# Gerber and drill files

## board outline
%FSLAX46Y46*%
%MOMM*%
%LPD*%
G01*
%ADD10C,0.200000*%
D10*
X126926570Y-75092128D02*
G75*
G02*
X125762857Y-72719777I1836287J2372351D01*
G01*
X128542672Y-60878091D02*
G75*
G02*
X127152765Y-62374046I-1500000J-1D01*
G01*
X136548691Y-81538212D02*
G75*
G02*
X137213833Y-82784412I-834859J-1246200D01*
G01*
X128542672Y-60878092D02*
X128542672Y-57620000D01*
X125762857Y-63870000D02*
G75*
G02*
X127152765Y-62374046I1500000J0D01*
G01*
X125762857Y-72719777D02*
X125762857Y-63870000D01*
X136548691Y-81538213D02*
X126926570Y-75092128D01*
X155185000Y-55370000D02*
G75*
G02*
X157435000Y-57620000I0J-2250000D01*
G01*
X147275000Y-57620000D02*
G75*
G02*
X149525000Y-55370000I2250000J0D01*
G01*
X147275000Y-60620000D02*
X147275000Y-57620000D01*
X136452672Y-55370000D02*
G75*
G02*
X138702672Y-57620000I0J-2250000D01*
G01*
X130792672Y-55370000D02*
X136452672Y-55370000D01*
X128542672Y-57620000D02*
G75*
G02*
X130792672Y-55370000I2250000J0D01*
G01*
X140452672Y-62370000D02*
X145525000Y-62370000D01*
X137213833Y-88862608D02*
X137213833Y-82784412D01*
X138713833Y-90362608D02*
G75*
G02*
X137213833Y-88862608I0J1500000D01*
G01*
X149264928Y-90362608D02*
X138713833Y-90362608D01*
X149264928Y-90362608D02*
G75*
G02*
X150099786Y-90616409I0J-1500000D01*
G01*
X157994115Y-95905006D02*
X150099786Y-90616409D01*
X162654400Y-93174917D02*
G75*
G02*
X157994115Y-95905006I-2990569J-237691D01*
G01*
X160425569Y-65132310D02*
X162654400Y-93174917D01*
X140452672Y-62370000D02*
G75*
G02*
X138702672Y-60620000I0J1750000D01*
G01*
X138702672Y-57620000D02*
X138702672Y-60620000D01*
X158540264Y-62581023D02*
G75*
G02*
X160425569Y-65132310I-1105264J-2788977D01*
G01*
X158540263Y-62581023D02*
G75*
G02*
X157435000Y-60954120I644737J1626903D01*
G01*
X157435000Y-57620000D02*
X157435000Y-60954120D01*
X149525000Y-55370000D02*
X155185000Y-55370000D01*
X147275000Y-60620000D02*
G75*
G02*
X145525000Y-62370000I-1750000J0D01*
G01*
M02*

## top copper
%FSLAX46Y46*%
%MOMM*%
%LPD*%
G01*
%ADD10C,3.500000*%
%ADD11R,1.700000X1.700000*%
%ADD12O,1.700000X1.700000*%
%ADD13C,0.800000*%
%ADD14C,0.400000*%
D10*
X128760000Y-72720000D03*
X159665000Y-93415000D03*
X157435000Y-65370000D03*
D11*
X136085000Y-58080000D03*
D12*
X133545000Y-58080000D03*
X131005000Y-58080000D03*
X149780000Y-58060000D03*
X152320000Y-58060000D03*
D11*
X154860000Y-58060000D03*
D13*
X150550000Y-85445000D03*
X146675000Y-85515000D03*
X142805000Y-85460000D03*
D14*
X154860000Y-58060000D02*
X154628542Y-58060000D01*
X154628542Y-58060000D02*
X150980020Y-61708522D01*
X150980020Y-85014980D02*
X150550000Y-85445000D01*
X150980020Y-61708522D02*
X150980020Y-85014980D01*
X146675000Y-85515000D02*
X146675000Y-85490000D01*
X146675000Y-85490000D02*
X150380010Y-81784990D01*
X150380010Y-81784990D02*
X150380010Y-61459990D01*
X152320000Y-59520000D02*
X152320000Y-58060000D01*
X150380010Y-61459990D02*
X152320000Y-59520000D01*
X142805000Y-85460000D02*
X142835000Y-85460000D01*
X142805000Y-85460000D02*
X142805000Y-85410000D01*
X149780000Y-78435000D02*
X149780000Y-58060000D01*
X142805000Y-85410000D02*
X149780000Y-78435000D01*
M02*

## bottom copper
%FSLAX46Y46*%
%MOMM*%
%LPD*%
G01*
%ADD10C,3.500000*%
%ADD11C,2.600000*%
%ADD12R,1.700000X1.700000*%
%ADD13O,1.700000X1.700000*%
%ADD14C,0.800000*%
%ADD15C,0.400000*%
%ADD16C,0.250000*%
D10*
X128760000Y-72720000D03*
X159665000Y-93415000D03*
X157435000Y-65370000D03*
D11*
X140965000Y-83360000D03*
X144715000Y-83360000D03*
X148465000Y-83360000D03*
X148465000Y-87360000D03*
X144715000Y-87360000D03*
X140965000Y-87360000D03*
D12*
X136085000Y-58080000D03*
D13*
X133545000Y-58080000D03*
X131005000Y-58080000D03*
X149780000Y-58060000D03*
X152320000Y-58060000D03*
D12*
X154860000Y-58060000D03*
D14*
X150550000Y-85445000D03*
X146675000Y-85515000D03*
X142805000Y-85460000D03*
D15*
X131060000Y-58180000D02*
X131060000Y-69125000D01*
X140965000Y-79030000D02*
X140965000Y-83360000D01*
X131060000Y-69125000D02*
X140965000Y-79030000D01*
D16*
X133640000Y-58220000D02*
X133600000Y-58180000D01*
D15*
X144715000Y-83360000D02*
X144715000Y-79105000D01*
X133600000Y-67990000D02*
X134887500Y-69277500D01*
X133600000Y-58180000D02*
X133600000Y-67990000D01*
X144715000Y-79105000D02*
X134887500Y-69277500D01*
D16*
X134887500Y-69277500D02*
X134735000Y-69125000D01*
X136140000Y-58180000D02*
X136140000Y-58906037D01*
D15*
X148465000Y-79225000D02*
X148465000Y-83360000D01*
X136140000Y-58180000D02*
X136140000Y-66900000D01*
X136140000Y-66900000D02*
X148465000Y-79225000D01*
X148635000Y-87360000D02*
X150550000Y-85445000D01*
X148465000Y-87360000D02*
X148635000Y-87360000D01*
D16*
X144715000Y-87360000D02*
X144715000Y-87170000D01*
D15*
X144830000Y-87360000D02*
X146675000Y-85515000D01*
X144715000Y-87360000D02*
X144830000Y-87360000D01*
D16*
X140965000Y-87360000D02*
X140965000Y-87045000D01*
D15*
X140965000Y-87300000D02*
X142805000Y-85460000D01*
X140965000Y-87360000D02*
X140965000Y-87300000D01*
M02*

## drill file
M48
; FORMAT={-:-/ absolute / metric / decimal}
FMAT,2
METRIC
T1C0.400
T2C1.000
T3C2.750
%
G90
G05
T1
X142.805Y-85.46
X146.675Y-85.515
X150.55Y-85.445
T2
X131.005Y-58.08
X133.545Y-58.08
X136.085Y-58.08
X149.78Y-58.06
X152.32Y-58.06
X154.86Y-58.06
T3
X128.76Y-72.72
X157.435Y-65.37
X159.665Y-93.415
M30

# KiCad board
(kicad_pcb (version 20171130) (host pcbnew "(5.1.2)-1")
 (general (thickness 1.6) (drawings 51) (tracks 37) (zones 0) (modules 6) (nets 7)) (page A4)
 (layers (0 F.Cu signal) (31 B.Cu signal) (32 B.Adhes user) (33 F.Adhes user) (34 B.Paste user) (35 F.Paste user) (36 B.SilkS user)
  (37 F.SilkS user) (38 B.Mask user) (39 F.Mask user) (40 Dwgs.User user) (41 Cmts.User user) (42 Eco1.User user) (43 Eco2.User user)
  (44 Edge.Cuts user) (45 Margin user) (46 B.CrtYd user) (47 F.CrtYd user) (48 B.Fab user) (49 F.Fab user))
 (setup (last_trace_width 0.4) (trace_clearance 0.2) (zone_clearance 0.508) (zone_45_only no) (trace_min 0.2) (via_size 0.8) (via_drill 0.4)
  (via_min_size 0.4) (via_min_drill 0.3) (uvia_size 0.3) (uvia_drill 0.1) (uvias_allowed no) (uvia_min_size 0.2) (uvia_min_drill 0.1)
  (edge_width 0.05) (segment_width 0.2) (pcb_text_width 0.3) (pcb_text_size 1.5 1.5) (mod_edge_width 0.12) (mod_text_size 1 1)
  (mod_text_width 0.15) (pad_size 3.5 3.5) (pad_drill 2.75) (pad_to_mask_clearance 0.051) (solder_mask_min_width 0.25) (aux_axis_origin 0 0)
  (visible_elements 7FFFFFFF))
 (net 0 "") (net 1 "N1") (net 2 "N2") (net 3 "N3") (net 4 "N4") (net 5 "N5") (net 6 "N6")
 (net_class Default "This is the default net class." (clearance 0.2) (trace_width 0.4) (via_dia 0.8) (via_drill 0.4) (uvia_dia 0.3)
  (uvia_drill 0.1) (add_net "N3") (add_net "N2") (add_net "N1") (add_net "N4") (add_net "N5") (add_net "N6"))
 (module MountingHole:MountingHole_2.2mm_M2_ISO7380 (layer F.Cu) (at 128.76 72.72)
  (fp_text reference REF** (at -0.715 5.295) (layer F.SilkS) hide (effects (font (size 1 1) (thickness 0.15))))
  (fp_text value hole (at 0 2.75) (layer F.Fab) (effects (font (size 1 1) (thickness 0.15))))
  (pad "" np_thru_hole circle (at 0 0) (size 3.5 3.5) (drill 2.75) (layers *.Cu *.Mask)))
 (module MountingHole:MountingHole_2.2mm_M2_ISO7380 (layer F.Cu) (at 159.665 93.415)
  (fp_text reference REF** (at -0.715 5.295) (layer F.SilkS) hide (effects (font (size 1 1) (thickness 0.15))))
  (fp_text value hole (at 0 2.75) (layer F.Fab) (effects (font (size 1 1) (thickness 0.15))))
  (pad "" np_thru_hole circle (at 0 0) (size 3.5 3.5) (drill 2.75) (layers *.Cu *.Mask)))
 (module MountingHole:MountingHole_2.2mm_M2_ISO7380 (layer F.Cu) (at 157.435 65.37)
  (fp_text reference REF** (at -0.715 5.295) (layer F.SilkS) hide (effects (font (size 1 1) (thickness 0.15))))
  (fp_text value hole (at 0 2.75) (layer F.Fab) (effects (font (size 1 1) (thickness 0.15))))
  (pad "" np_thru_hole circle (at 0 0) (size 3.5 3.5) (drill 2.75) (layers *.Cu *.Mask)))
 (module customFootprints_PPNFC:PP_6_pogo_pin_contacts (layer B.Cu) (at 148.465 83.36 180)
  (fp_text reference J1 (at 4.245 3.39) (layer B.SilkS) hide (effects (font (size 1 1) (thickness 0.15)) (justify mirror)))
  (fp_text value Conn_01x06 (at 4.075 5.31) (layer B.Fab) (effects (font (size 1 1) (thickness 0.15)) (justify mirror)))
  (pad 3 smd circle (at 7.5 0 180) (size 2.6 2.6) (layers B.Cu B.Paste B.Mask) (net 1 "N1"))
  (pad 2 smd circle (at 3.75 0 180) (size 2.6 2.6) (layers B.Cu B.Paste B.Mask) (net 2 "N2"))
  (pad 1 smd circle (at 0 0 180) (size 2.6 2.6) (layers B.Cu B.Paste B.Mask) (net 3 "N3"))
  (pad 4 smd circle (at 0 -4 180) (size 2.6 2.6) (layers B.Cu B.Paste B.Mask) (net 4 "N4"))
  (pad 5 smd circle (at 3.75 -4 180) (size 2.6 2.6) (layers B.Cu B.Paste B.Mask) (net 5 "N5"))
  (pad 6 smd circle (at 7.5 -4 180) (size 2.6 2.6) (layers B.Cu B.Paste B.Mask) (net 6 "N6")))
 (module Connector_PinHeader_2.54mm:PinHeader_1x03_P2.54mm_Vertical (layer F.Cu) (at 136.085 58.08 270)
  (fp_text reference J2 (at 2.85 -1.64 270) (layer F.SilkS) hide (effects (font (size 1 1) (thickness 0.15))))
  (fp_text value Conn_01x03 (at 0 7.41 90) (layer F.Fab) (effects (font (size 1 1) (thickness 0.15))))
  (pad 1 thru_hole rect (at 0 0 270) (size 1.7 1.7) (drill 1) (layers *.Cu *.Mask) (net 3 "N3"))
  (pad 2 thru_hole oval (at 0 2.54 270) (size 1.7 1.7) (drill 1) (layers *.Cu *.Mask) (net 2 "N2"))
  (pad 3 thru_hole oval (at 0 5.08 270) (size 1.7 1.7) (drill 1) (layers *.Cu *.Mask) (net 1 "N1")))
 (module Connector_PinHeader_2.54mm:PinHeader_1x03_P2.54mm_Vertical (layer F.Cu) (at 154.86 58.06 270)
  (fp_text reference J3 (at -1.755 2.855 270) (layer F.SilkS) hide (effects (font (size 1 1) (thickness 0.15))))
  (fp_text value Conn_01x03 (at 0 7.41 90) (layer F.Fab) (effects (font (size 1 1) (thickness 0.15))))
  (pad 3 thru_hole oval (at 0 5.08 270) (size 1.7 1.7) (drill 1) (layers *.Cu *.Mask) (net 6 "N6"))
  (pad 2 thru_hole oval (at 0 2.54 270) (size 1.7 1.7) (drill 1) (layers *.Cu *.Mask) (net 5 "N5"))
  (pad 1 thru_hole rect (at 0 0 270) (size 1.7 1.7) (drill 1) (layers *.Cu *.Mask) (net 4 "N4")))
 (gr_arc (start 128.762857 72.719777) (end 125.762857 72.719777) (angle -52.25880262) (layer Edge.Cuts) (width 0.2))
 (gr_arc (start 127.042672 60.878092) (end 127.152765 62.374046) (angle -85.79099191) (layer Edge.Cuts) (width 0.2))
 (gr_arc (start 135.713832 82.784412) (end 137.213833 82.784412) (angle -56.18093969) (layer Edge.Cuts) (width 0.2))
 (gr_line (start 128.542672 60.878092) (end 128.542672 57.62) (layer Edge.Cuts) (width 0.2))
 (gr_arc (start 127.262857 63.87) (end 127.152765 62.374046) (angle -85.79099191) (layer Edge.Cuts) (width 0.2))
 (gr_line (start 125.762857 72.719777) (end 125.762857 63.87) (layer Edge.Cuts) (width 0.2))
 (gr_line (start 136.548691 81.538213) (end 126.92657 75.092128) (layer Edge.Cuts) (width 0.2))
 (gr_arc (start 155.185 57.62) (end 157.435 57.62) (angle -90) (layer Edge.Cuts) (width 0.2))
 (gr_arc (start 149.525 57.62) (end 149.525 55.37) (angle -90) (layer Edge.Cuts) (width 0.2))
 (gr_line (start 147.275 60.62) (end 147.275 57.62) (layer Edge.Cuts) (width 0.2))
 (gr_arc (start 136.452672 57.62) (end 138.702672 57.62) (angle -90) (layer Edge.Cuts) (width 0.2))
 (gr_line (start 130.792672 55.37) (end 136.452672 55.37) (layer Edge.Cuts) (width 0.2))
 (gr_arc (start 130.792672 57.62) (end 130.792672 55.37) (angle -90) (layer Edge.Cuts) (width 0.2))
 (gr_line (start 140.452672 62.37) (end 145.525 62.37) (layer Edge.Cuts) (width 0.2))
 (gr_line (start 137.213833 88.862608) (end 137.213833 82.784412) (layer Edge.Cuts) (width 0.2))
 (gr_arc (start 138.713833 88.862608) (end 137.213833 88.862608) (angle -90) (layer Edge.Cuts) (width 0.2))
 (gr_line (start 149.264928 90.362608) (end 138.713833 90.362608) (layer Edge.Cuts) (width 0.2))
 (gr_arc (start 149.264928 91.862608) (end 150.099786 90.616409) (angle -33.81906031) (layer Edge.Cuts) (width 0.2))
 (gr_line (start 157.994115 95.905006) (end 150.099786 90.616409) (layer Edge.Cuts) (width 0.2))
 (gr_arc (start 159.663831 93.412608) (end 157.994115 95.905006) (angle -128.3633848) (layer Edge.Cuts) (width 0.2))
 (gr_line (start 160.425569 65.13231) (end 162.6544 93.174917) (layer Edge.Cuts) (width 0.2))
 (gr_arc (start 140.452672 60.62) (end 138.702672 60.62) (angle -90) (layer Edge.Cuts) (width 0.2))
 (gr_line (start 138.702672 57.62) (end 138.702672 60.62) (layer Edge.Cuts) (width 0.2))
 (gr_arc (start 157.435 65.37) (end 160.425569 65.13231) (angle -63.83740313) (layer Edge.Cuts) (width 0.2))
 (gr_arc (start 159.185 60.95412) (end 157.435 60.95412) (angle -68.38172758) (layer Edge.Cuts) (width 0.2))
 (gr_line (start 157.435 57.62) (end 157.435 60.95412) (layer Edge.Cuts) (width 0.2))
 (gr_line (start 149.525 55.37) (end 155.185 55.37) (layer Edge.Cuts) (width 0.2))
 (gr_arc (start 145.525 60.62) (end 145.525 62.37) (angle -90) (layer Edge.Cuts) (width 0.2))
 (segment (start 131.06 58.18) (end 131.06 69.125) (width 0.4) (layer B.Cu) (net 1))
 (segment (start 140.965 79.03) (end 140.965 83.36) (width 0.4) (layer B.Cu) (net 1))
 (segment (start 131.06 69.125) (end 140.965 79.03) (width 0.4) (layer B.Cu) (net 1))
 (segment (start 133.64 58.22) (end 133.6 58.18) (width 0.25) (layer B.Cu) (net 2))
 (segment (start 144.715 83.36) (end 144.715 79.105) (width 0.4) (layer B.Cu) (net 2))
 (segment (start 133.6 67.99) (end 134.8875 69.2775) (width 0.4) (layer B.Cu) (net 2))
 (segment (start 133.6 58.18) (end 133.6 67.99) (width 0.4) (layer B.Cu) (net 2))
 (segment (start 144.715 79.105) (end 134.8875 69.2775) (width 0.4) (layer B.Cu) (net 2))
 (segment (start 134.8875 69.2775) (end 134.735 69.125) (width 0.25) (layer B.Cu) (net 2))
 (segment (start 136.14 58.18) (end 136.14 58.906037) (width 0.25) (layer B.Cu) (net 3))
 (segment (start 148.465 79.225) (end 148.465 83.36) (width 0.4) (layer B.Cu) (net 3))
 (segment (start 136.14 58.18) (end 136.14 66.9) (width 0.4) (layer B.Cu) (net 3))
 (segment (start 136.14 66.9) (end 148.465 79.225) (width 0.4) (layer B.Cu) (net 3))
 (via (at 150.55 85.445) (size 0.8) (drill 0.4) (layers F.Cu B.Cu) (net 4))
 (segment (start 148.635 87.36) (end 150.55 85.445) (width 0.4) (layer B.Cu) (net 4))
 (segment (start 148.465 87.36) (end 148.635 87.36) (width 0.4) (layer B.Cu) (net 4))
 (segment (start 154.86 58.06) (end 154.628542 58.06) (width 0.4) (layer F.Cu) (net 4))
 (segment (start 154.628542 58.06) (end 150.98002 61.708522) (width 0.4) (layer F.Cu) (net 4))
 (segment (start 150.98002 85.01498) (end 150.55 85.445) (width 0.4) (layer F.Cu) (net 4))
 (segment (start 150.98002 61.708522) (end 150.98002 85.01498) (width 0.4) (layer F.Cu) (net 4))
 (via (at 146.675 85.515) (size 0.8) (drill 0.4) (layers F.Cu B.Cu) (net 5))
 (segment (start 144.715 87.36) (end 144.715 87.17) (width 0.25) (layer B.Cu) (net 5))
 (segment (start 144.83 87.36) (end 146.675 85.515) (width 0.4) (layer B.Cu) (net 5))
 (segment (start 144.715 87.36) (end 144.83 87.36) (width 0.4) (layer B.Cu) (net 5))
 (segment (start 146.675 85.515) (end 146.675 85.49) (width 0.4) (layer F.Cu) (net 5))
 (segment (start 146.675 85.49) (end 150.38001 81.78499) (width 0.4) (layer F.Cu) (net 5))
 (segment (start 150.38001 81.78499) (end 150.38001 61.45999) (width 0.4) (layer F.Cu) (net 5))
 (segment (start 152.32 59.52) (end 152.32 58.06) (width 0.4) (layer F.Cu) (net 5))
 (segment (start 150.38001 61.45999) (end 152.32 59.52) (width 0.4) (layer F.Cu) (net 5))
 (via (at 142.805 85.46) (size 0.8) (drill 0.4) (layers F.Cu B.Cu) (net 6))
 (segment (start 140.965 87.36) (end 140.965 87.045) (width 0.25) (layer B.Cu) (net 6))
 (segment (start 140.965 87.3) (end 142.805 85.46) (width 0.4) (layer B.Cu) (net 6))
 (segment (start 140.965 87.36) (end 140.965 87.3) (width 0.4) (layer B.Cu) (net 6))
 (segment (start 142.805 85.46) (end 142.835 85.46) (width 0.4) (layer F.Cu) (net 6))
 (segment (start 142.805 85.46) (end 142.805 85.41) (width 0.4) (layer F.Cu) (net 6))
 (segment (start 149.78 78.435) (end 149.78 58.06) (width 0.4) (layer F.Cu) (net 6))
 (segment (start 142.805 85.41) (end 149.78 78.435) (width 0.4) (layer F.Cu) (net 6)))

